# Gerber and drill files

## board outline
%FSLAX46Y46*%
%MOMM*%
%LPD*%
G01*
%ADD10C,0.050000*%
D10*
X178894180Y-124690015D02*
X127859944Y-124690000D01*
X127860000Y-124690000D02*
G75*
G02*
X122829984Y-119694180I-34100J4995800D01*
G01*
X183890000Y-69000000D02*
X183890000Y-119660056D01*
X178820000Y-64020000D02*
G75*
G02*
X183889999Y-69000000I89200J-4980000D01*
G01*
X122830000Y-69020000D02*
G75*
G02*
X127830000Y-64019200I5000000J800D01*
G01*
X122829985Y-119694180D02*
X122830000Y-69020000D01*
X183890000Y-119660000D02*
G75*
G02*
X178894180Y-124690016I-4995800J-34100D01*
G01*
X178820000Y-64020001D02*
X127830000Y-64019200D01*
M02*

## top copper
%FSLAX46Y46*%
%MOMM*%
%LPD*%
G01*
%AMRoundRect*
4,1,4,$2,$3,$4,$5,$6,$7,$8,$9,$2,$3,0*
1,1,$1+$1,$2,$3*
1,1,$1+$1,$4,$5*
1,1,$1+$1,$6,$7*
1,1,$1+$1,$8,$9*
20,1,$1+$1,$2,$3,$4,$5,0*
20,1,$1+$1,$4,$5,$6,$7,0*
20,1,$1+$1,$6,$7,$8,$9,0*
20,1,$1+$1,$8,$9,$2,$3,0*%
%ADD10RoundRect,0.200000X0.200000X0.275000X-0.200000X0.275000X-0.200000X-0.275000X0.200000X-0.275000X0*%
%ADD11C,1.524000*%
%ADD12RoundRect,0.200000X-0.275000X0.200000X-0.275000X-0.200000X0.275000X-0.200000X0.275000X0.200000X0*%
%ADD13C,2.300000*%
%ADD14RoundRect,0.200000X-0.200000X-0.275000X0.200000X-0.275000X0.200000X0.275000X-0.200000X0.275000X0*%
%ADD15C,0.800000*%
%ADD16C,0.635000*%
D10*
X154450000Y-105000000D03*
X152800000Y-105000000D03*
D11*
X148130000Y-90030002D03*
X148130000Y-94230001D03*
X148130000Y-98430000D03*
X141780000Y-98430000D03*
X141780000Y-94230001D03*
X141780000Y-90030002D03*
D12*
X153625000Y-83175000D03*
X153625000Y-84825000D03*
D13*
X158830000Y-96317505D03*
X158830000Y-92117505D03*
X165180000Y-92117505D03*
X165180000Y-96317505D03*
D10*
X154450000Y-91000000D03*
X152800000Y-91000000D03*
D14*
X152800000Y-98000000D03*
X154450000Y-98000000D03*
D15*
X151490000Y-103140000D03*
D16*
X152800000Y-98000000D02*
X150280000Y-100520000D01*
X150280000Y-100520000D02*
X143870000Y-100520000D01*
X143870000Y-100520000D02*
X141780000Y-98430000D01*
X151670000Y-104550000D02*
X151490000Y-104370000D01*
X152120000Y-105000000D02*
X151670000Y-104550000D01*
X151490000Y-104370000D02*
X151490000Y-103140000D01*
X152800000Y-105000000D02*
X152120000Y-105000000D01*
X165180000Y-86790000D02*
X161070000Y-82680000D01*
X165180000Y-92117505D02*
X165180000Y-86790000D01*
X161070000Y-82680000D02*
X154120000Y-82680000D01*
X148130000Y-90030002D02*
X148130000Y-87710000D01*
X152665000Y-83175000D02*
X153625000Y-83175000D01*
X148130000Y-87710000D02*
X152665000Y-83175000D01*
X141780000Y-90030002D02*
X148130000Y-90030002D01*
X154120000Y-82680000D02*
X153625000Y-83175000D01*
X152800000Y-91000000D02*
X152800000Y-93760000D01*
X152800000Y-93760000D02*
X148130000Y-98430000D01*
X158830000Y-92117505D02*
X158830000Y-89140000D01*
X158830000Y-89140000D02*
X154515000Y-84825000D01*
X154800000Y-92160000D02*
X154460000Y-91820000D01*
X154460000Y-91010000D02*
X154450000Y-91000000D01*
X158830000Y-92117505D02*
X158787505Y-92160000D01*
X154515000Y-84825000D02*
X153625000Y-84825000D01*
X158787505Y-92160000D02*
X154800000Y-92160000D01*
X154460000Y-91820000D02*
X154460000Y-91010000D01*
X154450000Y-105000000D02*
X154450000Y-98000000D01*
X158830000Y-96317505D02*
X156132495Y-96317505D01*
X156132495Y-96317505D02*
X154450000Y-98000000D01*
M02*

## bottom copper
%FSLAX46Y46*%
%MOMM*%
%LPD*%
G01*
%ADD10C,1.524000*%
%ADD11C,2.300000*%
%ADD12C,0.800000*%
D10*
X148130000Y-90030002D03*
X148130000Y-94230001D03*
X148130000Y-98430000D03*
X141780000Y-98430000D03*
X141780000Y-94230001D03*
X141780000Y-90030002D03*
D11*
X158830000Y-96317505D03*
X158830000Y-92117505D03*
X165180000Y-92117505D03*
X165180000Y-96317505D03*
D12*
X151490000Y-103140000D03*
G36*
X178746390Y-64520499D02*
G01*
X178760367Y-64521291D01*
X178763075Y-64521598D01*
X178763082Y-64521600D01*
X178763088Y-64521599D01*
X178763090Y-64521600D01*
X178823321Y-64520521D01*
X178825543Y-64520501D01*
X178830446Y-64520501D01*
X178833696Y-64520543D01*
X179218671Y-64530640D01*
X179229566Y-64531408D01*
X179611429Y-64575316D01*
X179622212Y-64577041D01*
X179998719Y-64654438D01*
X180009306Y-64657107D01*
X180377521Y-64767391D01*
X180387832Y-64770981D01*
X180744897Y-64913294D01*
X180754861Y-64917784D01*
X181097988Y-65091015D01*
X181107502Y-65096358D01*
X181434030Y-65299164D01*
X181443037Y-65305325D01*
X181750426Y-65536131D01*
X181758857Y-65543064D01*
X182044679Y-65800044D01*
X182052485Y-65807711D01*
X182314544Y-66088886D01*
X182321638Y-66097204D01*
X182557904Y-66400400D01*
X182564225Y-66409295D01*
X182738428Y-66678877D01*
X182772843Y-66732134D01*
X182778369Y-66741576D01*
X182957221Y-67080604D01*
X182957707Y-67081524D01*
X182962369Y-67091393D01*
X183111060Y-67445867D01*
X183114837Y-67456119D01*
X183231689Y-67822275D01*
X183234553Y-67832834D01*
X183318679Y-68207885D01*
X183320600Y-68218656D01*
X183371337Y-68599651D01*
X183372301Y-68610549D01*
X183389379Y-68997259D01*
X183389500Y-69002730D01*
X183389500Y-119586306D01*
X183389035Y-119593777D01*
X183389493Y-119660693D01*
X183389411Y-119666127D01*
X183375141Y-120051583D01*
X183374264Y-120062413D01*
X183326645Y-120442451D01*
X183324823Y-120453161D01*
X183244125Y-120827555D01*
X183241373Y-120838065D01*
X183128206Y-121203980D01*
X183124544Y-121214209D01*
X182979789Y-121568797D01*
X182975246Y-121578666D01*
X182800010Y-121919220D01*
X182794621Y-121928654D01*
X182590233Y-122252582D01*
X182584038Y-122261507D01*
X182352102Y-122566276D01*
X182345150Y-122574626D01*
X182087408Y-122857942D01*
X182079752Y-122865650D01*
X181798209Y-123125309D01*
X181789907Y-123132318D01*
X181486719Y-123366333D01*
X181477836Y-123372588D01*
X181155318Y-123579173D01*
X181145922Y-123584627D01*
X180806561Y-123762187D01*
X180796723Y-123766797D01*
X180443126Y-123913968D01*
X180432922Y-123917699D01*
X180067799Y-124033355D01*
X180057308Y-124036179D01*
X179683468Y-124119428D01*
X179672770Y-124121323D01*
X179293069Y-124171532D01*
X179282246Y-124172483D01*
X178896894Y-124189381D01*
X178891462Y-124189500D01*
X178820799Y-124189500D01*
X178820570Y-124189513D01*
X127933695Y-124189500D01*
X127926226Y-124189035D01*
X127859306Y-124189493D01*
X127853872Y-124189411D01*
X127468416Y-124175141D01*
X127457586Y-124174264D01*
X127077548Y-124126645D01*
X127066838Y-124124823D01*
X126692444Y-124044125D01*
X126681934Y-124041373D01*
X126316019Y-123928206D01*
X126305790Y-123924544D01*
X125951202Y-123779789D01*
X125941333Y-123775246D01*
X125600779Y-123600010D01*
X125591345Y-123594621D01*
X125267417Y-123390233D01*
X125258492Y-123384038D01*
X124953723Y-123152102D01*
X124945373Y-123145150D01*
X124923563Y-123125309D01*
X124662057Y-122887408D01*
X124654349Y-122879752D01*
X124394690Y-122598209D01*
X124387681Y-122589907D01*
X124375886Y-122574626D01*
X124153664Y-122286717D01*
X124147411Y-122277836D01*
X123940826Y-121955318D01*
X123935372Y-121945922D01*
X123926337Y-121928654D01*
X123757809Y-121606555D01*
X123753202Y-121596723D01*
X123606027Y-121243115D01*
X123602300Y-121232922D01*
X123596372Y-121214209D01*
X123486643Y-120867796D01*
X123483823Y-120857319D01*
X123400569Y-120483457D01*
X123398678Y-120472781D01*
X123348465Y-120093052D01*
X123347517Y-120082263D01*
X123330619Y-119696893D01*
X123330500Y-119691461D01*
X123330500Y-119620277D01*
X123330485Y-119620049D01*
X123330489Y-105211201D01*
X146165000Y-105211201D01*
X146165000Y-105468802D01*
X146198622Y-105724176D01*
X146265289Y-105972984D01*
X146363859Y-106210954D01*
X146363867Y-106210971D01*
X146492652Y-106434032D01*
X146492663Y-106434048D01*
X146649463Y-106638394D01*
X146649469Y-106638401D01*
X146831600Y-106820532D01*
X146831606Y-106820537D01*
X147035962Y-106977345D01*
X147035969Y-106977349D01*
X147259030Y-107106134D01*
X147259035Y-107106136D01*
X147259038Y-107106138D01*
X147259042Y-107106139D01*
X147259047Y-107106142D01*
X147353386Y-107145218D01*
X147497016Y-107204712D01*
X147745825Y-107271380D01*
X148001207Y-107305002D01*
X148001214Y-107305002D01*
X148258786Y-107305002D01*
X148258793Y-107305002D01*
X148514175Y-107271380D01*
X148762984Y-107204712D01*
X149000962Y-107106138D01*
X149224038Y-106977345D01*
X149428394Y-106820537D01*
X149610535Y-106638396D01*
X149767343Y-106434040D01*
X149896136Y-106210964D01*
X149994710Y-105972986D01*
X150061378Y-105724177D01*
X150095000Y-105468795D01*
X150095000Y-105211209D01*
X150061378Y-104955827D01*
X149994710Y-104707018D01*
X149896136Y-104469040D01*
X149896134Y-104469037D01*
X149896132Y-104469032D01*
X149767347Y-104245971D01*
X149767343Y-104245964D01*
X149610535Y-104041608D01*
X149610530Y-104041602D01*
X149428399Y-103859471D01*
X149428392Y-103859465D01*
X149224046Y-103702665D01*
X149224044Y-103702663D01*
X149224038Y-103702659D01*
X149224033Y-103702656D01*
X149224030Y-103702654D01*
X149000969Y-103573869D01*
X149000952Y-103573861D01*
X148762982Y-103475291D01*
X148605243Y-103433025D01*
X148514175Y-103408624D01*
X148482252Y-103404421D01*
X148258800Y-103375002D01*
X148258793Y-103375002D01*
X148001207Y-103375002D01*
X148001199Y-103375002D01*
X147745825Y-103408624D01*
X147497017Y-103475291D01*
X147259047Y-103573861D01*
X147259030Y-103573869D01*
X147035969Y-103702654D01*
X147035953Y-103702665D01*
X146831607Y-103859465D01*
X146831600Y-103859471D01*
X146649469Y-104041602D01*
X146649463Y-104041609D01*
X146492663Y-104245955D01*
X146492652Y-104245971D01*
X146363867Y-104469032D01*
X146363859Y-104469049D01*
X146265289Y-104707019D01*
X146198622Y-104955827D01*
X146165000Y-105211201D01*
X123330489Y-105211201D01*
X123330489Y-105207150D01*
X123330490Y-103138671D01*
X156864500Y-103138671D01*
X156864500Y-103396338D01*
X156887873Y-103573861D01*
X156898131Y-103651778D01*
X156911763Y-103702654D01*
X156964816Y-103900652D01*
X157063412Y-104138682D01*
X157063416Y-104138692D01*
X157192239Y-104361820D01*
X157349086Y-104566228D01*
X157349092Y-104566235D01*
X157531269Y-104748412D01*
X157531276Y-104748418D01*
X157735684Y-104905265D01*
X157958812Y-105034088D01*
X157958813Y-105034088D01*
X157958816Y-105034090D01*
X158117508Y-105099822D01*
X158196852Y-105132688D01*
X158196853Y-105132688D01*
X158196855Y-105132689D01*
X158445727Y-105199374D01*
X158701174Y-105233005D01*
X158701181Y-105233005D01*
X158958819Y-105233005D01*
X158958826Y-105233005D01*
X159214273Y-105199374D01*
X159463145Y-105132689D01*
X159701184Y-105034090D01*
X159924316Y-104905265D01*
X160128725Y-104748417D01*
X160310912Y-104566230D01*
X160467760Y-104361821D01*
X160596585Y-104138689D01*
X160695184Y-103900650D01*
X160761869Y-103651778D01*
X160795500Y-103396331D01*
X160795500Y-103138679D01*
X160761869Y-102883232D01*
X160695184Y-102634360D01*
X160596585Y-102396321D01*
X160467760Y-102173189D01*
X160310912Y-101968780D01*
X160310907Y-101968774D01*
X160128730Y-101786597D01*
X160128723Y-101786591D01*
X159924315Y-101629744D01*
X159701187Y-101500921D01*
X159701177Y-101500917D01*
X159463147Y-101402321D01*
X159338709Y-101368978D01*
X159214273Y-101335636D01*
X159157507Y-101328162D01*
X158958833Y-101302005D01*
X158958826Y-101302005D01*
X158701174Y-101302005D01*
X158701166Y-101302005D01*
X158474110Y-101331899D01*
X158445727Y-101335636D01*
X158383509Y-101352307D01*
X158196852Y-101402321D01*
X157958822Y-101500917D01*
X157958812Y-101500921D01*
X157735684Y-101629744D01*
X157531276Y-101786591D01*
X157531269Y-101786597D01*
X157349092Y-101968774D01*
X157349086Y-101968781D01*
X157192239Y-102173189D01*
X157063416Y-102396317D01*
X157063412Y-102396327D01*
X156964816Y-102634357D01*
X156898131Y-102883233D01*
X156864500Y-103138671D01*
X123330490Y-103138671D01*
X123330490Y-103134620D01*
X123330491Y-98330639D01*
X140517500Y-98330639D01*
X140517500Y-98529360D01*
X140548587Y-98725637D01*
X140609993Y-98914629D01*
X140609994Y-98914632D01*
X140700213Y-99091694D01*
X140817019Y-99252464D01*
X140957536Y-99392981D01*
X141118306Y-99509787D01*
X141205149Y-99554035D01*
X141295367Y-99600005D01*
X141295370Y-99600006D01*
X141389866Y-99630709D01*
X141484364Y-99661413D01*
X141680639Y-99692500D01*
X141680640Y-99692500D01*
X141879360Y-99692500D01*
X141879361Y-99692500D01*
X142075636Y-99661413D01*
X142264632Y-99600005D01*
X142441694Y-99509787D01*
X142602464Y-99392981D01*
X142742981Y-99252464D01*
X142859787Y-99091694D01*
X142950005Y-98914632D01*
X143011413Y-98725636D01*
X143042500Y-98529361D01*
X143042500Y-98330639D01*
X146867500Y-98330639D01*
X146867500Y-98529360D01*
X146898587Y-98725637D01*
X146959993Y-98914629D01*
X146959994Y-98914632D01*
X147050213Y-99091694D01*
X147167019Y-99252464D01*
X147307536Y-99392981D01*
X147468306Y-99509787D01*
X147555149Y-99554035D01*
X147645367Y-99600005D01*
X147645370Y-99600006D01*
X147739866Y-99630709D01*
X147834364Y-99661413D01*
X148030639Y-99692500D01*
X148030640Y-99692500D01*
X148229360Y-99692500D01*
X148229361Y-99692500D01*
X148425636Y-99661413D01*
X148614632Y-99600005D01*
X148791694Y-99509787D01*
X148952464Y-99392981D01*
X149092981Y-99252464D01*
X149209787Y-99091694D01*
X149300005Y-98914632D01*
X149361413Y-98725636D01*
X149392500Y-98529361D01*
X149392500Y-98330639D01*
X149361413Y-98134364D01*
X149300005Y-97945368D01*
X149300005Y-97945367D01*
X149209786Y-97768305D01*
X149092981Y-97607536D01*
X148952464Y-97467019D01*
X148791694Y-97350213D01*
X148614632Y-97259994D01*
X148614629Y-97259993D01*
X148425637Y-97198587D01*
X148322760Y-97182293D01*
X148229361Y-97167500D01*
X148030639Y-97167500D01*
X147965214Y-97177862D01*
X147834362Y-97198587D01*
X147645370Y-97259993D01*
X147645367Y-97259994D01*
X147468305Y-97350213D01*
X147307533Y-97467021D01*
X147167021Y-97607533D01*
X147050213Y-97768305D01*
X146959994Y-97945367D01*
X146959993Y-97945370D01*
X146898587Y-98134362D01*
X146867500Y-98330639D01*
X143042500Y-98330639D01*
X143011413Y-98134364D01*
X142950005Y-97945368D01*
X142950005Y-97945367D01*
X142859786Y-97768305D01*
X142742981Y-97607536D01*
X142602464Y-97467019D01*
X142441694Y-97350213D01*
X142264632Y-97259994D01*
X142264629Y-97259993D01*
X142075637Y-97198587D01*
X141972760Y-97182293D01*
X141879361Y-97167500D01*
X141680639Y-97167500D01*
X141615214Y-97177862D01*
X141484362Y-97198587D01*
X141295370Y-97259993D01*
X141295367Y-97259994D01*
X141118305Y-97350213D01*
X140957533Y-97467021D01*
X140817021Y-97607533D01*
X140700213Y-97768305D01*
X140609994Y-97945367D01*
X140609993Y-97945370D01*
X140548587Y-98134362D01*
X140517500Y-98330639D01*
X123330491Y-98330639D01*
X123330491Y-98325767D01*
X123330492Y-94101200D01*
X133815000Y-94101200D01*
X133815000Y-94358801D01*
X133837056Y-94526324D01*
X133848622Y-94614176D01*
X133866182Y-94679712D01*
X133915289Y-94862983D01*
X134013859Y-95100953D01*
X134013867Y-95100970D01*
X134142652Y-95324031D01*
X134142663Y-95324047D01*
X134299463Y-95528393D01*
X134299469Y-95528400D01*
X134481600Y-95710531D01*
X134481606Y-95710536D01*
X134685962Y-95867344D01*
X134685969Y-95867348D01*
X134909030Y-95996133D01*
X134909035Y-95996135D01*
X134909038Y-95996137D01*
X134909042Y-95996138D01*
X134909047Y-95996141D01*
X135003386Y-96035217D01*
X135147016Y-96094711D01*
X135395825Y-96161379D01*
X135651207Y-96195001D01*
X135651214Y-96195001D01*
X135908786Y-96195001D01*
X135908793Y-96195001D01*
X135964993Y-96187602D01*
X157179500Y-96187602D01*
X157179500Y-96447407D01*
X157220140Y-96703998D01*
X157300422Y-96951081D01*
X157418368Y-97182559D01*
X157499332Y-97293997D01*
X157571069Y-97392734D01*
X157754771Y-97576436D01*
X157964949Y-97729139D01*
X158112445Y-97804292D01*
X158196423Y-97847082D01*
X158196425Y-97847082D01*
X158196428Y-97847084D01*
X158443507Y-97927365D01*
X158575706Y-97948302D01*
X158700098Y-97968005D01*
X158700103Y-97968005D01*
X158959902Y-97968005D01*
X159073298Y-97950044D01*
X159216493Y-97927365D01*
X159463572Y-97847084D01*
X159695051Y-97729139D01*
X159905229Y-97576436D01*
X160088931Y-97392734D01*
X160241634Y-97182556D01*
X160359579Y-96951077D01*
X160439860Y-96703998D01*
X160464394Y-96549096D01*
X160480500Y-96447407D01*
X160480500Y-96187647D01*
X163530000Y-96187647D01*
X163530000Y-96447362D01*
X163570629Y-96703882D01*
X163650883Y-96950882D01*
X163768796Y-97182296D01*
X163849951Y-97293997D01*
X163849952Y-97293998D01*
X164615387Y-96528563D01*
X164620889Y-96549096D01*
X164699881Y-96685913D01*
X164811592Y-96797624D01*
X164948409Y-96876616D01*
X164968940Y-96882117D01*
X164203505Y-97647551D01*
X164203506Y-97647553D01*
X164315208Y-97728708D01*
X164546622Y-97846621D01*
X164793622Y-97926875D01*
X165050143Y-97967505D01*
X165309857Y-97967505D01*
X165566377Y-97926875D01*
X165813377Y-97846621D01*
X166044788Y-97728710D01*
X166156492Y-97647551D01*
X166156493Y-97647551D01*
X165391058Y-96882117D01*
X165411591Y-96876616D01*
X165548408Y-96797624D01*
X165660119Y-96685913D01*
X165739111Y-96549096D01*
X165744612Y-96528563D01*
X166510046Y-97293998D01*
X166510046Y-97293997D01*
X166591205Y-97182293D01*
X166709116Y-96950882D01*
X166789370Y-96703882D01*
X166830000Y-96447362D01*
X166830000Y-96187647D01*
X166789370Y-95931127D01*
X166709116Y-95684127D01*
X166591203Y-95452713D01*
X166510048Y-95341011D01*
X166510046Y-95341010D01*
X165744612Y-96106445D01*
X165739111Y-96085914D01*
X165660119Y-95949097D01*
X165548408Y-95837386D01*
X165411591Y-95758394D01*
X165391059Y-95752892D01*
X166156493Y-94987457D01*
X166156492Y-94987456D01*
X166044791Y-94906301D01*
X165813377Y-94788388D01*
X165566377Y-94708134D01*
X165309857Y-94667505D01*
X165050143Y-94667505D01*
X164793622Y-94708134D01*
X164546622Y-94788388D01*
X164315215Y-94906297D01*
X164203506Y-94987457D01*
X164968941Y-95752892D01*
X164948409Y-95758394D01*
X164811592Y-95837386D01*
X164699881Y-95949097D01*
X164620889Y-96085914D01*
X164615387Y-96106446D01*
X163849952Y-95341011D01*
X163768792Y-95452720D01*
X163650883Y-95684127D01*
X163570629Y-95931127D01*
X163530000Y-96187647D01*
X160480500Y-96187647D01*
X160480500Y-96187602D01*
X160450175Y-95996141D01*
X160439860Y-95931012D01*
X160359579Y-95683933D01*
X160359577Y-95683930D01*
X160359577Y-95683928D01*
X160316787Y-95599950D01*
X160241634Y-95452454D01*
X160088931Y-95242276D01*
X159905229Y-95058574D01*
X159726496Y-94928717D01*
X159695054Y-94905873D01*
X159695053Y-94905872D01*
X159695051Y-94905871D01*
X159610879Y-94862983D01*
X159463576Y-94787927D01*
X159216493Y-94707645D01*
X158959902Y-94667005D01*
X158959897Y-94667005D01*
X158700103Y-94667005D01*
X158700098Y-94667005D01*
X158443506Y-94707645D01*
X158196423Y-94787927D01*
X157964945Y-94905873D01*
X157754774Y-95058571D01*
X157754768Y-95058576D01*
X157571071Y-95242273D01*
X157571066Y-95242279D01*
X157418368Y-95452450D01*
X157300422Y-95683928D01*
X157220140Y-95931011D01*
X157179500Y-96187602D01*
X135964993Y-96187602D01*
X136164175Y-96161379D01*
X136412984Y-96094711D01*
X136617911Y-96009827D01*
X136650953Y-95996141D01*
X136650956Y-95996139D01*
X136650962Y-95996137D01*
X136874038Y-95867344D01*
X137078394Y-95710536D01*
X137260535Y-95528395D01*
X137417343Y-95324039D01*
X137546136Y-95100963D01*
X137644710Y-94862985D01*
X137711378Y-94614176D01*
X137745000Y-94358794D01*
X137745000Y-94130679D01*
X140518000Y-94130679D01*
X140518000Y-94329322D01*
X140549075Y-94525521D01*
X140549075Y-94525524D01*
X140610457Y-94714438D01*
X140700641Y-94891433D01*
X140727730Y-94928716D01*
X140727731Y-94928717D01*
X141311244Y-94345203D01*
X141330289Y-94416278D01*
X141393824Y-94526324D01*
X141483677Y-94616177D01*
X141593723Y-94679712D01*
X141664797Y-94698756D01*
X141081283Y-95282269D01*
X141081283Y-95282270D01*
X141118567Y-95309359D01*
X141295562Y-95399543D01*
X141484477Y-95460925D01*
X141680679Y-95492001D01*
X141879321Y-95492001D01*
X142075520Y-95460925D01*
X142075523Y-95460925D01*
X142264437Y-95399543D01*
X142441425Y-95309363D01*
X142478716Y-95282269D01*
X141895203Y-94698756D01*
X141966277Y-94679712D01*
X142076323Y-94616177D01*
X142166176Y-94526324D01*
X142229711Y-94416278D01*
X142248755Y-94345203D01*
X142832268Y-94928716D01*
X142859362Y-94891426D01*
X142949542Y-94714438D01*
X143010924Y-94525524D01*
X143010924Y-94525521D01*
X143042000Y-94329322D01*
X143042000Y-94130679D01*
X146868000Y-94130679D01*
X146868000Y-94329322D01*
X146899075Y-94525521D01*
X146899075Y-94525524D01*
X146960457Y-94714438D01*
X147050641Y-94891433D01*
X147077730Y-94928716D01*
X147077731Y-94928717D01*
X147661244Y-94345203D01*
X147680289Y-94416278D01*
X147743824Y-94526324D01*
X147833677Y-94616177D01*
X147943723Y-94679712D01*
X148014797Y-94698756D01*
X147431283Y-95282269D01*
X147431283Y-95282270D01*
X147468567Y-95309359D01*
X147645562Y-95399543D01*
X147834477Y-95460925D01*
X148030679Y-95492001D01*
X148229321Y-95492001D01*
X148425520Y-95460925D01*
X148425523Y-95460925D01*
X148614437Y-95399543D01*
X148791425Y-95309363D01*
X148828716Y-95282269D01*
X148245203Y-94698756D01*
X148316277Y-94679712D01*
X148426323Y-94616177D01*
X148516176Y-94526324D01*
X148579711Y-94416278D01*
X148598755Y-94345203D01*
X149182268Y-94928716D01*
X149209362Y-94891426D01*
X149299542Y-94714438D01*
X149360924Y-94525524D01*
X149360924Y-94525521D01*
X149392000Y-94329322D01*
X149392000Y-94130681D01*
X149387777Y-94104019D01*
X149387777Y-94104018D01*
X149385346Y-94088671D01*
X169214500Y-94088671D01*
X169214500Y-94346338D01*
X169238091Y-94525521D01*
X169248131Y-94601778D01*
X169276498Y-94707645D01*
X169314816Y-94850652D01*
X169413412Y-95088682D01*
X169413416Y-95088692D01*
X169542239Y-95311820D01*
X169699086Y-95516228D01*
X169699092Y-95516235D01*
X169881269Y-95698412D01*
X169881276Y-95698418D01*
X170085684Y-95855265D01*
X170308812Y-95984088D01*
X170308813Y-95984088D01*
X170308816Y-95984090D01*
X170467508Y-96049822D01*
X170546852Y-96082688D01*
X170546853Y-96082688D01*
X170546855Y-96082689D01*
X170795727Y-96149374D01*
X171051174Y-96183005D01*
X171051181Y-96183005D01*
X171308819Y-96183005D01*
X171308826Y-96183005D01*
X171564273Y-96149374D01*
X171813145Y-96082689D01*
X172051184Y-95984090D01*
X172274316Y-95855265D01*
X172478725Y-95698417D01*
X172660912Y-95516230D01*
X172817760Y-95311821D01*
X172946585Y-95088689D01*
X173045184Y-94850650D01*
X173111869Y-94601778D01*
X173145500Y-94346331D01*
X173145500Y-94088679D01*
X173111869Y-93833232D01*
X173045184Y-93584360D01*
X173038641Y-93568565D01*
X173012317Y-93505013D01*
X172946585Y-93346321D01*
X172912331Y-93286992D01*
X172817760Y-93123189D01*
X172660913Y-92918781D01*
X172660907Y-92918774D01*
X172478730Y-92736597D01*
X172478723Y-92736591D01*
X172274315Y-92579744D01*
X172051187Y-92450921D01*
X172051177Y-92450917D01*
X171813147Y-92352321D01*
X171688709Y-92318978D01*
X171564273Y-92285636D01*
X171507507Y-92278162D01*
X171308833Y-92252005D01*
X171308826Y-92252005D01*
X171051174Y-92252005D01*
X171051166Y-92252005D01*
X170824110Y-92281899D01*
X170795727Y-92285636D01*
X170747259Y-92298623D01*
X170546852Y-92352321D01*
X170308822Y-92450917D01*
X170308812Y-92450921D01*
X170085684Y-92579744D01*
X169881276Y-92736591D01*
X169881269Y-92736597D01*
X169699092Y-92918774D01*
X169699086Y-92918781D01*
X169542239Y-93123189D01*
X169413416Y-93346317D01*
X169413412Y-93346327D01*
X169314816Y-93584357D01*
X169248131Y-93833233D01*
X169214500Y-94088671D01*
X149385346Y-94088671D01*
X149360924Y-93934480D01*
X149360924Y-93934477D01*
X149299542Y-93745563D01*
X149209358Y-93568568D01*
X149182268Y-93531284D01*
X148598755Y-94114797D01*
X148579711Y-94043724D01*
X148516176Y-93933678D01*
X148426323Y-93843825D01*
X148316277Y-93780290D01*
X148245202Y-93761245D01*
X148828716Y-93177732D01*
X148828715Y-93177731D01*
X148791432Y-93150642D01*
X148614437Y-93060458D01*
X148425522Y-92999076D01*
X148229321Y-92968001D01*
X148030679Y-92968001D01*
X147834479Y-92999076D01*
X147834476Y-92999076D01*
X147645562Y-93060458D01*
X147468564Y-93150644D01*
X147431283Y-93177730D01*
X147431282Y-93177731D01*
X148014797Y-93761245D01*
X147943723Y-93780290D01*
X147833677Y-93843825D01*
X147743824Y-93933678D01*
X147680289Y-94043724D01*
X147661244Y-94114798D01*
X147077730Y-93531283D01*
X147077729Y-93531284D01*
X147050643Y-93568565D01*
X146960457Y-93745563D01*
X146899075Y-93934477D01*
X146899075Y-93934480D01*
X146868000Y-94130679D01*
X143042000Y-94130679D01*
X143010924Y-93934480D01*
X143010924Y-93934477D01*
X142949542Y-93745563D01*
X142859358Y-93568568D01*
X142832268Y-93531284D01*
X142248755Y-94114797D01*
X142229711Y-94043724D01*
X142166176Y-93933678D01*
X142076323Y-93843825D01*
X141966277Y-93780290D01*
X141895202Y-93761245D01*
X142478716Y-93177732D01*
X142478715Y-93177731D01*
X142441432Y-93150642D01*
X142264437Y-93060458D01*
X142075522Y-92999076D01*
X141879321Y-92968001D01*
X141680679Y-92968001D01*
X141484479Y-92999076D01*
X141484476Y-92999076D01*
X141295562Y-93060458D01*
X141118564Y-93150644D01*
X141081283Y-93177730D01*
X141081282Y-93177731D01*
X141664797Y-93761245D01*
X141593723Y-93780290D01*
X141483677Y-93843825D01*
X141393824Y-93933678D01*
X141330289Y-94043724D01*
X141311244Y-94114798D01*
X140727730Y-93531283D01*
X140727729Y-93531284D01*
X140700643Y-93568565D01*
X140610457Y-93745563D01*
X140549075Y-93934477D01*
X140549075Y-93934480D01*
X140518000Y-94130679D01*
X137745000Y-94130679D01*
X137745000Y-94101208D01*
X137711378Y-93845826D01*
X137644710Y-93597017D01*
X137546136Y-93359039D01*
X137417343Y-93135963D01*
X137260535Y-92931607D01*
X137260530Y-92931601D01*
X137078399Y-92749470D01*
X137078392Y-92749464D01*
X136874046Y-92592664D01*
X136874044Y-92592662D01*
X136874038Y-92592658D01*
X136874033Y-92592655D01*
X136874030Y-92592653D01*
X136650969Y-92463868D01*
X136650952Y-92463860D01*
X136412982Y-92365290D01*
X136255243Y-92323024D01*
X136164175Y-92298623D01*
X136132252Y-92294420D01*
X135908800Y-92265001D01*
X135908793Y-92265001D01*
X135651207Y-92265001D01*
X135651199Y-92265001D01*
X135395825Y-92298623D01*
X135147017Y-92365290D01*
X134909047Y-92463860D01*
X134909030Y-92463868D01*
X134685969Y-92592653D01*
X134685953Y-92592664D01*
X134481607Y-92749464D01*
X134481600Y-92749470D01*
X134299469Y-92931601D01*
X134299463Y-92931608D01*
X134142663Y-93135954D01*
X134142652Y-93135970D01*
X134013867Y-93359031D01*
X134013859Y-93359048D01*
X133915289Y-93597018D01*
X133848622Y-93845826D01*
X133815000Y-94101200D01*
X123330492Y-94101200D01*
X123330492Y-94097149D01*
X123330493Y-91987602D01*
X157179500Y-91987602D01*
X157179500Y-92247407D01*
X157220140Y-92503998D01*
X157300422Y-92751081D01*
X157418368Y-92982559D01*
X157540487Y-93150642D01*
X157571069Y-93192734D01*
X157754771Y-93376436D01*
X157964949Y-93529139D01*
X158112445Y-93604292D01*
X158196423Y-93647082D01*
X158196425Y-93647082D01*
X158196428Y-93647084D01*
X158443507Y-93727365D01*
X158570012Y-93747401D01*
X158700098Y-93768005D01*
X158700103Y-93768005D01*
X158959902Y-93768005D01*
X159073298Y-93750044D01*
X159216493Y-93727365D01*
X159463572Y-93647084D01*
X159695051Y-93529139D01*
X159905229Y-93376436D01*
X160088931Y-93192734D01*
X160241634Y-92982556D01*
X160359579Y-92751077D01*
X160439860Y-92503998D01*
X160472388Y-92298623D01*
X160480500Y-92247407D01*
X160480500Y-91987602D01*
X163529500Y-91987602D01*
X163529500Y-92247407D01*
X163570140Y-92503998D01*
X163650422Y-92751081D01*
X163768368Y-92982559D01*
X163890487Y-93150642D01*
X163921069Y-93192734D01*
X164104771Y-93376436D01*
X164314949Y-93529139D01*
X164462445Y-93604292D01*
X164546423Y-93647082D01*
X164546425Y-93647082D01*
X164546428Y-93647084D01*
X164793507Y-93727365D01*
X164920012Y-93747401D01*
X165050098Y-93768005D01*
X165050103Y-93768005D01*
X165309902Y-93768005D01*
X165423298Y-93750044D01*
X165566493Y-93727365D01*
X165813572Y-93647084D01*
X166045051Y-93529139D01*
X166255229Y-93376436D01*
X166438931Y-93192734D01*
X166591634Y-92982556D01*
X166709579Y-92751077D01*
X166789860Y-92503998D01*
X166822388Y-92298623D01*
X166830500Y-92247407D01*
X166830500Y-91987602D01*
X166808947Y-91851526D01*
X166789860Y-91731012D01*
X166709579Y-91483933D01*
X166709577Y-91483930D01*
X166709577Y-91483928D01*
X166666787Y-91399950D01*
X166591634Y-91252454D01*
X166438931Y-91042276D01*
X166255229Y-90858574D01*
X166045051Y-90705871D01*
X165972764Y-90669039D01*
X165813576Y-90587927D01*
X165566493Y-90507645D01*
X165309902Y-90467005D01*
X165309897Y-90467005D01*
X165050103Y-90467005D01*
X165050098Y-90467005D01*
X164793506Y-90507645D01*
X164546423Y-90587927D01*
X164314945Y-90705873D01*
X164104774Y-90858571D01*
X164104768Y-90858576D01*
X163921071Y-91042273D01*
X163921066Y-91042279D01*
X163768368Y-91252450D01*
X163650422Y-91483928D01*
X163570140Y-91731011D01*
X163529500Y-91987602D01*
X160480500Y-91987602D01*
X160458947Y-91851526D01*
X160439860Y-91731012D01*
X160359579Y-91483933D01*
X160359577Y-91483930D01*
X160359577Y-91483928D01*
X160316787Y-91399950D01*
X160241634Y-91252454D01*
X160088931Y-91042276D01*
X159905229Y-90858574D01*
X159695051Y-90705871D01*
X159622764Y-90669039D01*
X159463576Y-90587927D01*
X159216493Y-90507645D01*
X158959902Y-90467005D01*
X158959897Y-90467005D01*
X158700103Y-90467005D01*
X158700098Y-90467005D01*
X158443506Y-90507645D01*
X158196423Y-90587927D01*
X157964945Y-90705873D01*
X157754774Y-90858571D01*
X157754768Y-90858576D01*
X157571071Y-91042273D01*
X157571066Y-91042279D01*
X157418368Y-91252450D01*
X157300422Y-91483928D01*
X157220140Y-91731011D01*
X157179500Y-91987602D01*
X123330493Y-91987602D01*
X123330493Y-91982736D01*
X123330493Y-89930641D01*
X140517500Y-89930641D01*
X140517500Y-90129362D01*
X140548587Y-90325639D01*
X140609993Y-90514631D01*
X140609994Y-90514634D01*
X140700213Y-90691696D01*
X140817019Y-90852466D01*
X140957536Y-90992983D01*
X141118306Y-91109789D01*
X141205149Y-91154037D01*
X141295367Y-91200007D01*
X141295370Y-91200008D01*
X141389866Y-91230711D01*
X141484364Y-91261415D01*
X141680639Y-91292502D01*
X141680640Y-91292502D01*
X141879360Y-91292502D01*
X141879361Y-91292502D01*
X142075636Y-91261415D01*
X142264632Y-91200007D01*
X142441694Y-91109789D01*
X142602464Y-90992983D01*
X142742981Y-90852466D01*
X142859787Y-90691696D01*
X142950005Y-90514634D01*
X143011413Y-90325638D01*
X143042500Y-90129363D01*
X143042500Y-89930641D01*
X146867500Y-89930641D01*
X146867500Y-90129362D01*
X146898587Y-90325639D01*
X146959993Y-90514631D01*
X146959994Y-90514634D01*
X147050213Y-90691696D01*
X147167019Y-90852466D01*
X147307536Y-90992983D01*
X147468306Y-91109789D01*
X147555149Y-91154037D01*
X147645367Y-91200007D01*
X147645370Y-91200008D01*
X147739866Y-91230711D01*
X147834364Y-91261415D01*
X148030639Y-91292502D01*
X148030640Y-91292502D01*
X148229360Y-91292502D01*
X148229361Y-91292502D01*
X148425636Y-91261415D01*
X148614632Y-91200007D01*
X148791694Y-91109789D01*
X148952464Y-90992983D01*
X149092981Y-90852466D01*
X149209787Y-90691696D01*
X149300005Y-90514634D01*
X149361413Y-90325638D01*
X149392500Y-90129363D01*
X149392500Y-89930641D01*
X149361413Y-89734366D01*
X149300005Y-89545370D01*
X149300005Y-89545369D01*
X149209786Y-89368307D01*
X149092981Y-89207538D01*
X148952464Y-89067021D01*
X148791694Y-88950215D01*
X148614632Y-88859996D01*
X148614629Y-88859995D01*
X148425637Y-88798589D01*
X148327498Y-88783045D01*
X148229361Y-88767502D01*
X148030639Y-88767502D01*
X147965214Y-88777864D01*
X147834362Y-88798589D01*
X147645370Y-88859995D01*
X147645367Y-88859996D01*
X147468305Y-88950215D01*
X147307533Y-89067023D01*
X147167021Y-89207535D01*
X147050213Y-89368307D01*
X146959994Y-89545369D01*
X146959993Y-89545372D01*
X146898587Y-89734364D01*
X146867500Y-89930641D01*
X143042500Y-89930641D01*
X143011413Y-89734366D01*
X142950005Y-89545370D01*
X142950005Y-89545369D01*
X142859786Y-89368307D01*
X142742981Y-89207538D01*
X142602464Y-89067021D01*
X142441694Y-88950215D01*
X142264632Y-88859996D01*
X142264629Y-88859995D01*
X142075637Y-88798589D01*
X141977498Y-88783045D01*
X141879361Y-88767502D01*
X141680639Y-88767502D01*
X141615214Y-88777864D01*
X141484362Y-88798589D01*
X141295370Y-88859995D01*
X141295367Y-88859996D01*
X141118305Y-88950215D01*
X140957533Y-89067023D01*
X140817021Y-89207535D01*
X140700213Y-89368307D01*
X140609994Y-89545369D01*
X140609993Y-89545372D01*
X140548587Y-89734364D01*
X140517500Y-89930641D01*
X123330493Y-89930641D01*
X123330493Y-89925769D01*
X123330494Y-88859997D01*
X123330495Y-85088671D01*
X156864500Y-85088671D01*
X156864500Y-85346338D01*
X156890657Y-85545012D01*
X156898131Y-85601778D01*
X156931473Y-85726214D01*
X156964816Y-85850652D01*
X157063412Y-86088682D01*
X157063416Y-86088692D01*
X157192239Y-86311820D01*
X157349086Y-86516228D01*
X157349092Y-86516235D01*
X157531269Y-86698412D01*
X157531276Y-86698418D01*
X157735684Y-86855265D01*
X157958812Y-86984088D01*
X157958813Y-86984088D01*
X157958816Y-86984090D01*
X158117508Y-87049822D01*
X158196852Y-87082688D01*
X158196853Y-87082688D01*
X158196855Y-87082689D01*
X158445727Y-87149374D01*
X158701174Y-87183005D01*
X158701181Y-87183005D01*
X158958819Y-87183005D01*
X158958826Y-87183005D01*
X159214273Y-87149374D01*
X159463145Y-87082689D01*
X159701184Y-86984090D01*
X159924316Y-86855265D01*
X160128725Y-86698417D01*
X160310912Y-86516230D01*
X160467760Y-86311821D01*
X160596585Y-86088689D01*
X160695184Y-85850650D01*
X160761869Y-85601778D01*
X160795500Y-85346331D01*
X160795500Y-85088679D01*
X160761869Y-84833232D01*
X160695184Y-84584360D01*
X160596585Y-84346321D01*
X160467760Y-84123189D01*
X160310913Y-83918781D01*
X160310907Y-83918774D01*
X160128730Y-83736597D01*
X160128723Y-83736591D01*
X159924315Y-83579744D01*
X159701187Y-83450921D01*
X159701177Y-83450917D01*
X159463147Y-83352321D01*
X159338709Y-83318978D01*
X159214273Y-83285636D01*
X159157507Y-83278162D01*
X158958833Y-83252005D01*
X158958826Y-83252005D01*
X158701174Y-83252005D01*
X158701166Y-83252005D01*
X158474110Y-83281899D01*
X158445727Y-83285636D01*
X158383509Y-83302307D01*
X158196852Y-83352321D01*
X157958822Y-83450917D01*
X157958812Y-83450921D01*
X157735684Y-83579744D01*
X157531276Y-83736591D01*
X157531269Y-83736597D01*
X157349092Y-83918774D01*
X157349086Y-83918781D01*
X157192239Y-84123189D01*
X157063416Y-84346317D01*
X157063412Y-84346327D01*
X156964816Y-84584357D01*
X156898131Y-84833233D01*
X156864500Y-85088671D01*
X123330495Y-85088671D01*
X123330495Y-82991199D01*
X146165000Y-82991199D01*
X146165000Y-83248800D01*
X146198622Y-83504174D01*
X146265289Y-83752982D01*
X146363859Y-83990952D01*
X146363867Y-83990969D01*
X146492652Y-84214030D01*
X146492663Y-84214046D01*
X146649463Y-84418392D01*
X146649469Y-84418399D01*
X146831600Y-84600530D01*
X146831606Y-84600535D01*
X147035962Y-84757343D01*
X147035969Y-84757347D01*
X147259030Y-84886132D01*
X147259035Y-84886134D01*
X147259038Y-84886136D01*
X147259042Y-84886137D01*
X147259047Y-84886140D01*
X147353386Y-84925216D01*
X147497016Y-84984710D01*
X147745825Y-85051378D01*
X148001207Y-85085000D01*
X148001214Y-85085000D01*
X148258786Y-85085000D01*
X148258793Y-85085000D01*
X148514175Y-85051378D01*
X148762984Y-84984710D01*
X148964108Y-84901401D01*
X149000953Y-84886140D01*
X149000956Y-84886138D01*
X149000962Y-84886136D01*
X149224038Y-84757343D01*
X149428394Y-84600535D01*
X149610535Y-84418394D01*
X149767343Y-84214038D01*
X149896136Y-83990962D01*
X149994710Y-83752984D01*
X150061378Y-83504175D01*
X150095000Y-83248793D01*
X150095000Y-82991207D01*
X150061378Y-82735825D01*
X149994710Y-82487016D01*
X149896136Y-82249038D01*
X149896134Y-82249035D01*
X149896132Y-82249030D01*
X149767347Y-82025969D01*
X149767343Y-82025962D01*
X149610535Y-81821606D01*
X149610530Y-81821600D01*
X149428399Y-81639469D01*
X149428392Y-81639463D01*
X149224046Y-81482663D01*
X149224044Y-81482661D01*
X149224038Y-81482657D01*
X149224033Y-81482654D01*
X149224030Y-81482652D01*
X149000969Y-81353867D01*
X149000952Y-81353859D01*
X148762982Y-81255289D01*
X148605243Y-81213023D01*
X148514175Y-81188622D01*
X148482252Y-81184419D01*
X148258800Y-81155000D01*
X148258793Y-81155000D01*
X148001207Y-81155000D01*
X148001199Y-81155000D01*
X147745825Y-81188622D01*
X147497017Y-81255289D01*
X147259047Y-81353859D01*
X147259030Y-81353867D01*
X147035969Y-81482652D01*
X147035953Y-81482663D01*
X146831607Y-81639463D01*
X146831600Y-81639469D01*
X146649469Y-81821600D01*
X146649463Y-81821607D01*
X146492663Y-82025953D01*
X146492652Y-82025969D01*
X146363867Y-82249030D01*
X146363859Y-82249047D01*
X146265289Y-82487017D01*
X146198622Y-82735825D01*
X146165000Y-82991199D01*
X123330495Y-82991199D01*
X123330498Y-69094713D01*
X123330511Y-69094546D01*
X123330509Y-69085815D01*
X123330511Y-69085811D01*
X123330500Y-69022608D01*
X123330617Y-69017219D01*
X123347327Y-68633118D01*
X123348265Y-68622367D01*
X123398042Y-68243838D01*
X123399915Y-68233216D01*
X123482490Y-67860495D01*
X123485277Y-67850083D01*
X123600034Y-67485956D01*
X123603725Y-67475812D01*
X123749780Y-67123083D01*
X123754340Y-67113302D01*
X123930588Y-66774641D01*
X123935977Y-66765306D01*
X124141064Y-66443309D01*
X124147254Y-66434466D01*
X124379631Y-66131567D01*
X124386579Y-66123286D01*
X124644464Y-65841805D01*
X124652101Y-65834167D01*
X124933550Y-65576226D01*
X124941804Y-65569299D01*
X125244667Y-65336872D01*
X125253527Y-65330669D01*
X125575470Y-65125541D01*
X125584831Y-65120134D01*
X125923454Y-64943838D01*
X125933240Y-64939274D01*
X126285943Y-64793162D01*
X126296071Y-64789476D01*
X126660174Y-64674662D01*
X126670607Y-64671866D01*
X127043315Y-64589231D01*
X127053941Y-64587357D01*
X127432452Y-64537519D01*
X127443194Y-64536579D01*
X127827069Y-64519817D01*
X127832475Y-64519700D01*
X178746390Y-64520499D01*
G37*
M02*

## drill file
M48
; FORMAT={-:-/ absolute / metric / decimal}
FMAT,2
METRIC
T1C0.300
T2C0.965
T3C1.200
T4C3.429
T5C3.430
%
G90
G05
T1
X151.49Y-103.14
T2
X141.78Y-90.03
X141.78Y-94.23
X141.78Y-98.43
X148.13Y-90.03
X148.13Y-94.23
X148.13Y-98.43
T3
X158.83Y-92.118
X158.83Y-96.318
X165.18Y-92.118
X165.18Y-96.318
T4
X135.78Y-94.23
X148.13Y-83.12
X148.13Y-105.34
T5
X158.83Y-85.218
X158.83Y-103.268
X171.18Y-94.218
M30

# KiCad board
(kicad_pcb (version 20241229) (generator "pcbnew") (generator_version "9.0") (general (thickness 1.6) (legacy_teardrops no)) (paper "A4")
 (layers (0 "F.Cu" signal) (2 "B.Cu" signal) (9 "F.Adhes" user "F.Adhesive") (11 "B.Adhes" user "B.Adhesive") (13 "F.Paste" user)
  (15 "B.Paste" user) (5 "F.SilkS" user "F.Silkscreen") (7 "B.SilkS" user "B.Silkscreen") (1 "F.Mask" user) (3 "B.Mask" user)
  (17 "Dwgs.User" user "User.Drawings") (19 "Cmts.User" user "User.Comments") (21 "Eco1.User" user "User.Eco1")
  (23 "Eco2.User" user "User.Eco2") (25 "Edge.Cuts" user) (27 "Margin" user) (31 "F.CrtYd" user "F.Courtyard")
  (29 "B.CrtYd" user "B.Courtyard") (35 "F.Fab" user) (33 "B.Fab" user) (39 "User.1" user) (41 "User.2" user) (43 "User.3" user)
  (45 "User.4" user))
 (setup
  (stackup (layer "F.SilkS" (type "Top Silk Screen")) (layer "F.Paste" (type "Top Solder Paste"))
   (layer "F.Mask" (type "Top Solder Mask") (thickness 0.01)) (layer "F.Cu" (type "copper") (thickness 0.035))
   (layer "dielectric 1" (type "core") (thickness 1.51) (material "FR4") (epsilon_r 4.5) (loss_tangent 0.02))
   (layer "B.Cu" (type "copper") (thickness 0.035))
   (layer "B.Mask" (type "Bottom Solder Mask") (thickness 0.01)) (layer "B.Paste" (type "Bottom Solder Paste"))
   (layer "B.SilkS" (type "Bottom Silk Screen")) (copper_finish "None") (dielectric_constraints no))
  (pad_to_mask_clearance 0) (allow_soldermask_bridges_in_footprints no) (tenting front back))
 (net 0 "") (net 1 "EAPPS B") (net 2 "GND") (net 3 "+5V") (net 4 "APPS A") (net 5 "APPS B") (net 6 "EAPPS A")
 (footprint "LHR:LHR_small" (layer "F.Cu") (at 172.32 118.24)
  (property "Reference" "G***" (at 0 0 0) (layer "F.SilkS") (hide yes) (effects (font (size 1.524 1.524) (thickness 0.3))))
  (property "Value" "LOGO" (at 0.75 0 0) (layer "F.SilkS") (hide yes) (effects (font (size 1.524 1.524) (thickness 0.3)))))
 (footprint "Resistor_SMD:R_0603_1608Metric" (layer "F.Cu") (at 153.625 105 180)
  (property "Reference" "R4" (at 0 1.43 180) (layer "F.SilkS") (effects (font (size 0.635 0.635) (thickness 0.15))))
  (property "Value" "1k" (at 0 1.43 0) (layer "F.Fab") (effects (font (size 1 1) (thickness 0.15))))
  (pad "1" smd roundrect (at -0.825 0 180) (size 0.8 0.95) (layers "F.Cu" "F.Mask" "F.Paste") (roundrect_rratio 0.25) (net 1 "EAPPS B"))
  (pad "2" smd roundrect (at 0.825 0 180) (size 0.8 0.95) (layers "F.Cu" "F.Mask" "F.Paste") (roundrect_rratio 0.25) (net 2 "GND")))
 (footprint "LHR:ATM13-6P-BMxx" (layer "F.Cu") (at 148.13 90.030002 -90)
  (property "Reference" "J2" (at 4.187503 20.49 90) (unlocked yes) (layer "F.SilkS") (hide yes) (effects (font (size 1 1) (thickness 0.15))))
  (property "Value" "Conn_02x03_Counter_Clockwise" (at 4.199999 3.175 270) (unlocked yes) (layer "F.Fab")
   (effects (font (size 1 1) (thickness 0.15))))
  (pad "" np_thru_hole circle (at -6.910002 0 270) (size 3.937 3.937) (drill 3.429) (layers))
  (pad "" np_thru_hole circle (at 4.199999 12.35 270) (size 3.937 3.937) (drill 3.429) (layers))
  (pad "" np_thru_hole circle (at 15.31 0 270) (size 3.937 3.937) (drill 3.429) (layers))
  (pad "1" thru_hole circle (at 0 0 270) (size 1.524 1.524) (drill 0.9652) (layers "*.Cu" "*.Mask") (remove_unused_layers no) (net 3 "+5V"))
  (pad "2" thru_hole circle (at 4.199999 0 270) (size 1.524 1.524) (drill 0.9652) (layers "*.Cu" "*.Mask") (remove_unused_layers no)
   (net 2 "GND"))
  (pad "3" thru_hole circle (at 8.399998 0 270) (size 1.524 1.524) (drill 0.9652) (layers "*.Cu" "*.Mask") (remove_unused_layers no)
   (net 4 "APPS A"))
  (pad "4" thru_hole circle (at 8.399998 6.35 270) (size 1.524 1.524) (drill 0.9652) (layers "*.Cu" "*.Mask") (remove_unused_layers no)
   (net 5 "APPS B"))
  (pad "5" thru_hole circle (at 4.199999 6.35 270) (size 1.524 1.524) (drill 0.9652) (layers "*.Cu" "*.Mask") (remove_unused_layers no)
   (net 2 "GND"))
  (pad "6" thru_hole circle (at 0 6.35 270) (size 1.524 1.524) (drill 0.9652) (layers "*.Cu" "*.Mask") (remove_unused_layers no)
   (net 3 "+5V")))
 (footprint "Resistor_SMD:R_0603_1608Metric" (layer "F.Cu") (at 153.625 84 -90)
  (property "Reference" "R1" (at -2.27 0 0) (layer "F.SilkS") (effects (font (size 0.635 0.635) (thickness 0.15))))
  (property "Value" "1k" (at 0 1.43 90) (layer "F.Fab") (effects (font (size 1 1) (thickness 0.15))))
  (pad "1" smd roundrect (at -0.825 0 270) (size 0.8 0.95) (layers "F.Cu" "F.Mask" "F.Paste") (roundrect_rratio 0.25) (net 3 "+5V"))
  (pad "2" smd roundrect (at 0.825 0 270) (size 0.8 0.95) (layers "F.Cu" "F.Mask" "F.Paste") (roundrect_rratio 0.25) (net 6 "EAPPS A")))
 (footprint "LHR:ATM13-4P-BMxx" (layer "F.Cu") (at 164.08 94.217505 -90)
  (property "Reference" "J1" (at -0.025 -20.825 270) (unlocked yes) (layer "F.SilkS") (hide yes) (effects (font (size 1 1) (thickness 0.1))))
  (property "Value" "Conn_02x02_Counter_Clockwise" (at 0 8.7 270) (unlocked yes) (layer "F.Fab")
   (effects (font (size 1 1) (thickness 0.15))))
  (pad "" np_thru_hole circle (at -9 5.25 270) (size 3.43 3.43) (drill 3.43) (layers "*.Cu" "*.Mask"))
  (pad "" np_thru_hole circle (at 0 -7.1 270) (size 3.43 3.43) (drill 3.43) (layers "*.Cu" "*.Mask"))
  (pad "" np_thru_hole circle (at 9.05 5.25 270) (size 3.43 3.43) (drill 3.43) (layers "*.Cu" "*.Mask"))
  (pad "1" thru_hole circle (at 2.1 5.25 270) (size 2.3 2.3) (drill 1.2) (layers "*.Cu" "*.Mask") (remove_unused_layers no)
   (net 1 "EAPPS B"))
  (pad "2" thru_hole circle (at -2.1 5.25 270) (size 2.3 2.3) (drill 1.2) (layers "*.Cu" "*.Mask") (remove_unused_layers no)
   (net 6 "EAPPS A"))
  (pad "3" thru_hole circle (at -2.1 -1.1 270) (size 2.3 2.3) (drill 1.2) (layers "*.Cu" "*.Mask") (remove_unused_layers no) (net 3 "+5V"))
  (pad "4" thru_hole circle (at 2.1 -1.1 270) (size 2.3 2.3) (drill 1.2) (layers "*.Cu" "*.Mask") (remove_unused_layers no) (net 2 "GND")))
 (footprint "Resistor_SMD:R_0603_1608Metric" (layer "F.Cu") (at 153.625 91 180)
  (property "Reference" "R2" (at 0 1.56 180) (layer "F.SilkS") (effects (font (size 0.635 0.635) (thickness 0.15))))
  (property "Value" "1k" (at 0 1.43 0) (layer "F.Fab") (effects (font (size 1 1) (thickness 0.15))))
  (pad "1" smd roundrect (at -0.825 0 180) (size 0.8 0.95) (layers "F.Cu" "F.Mask" "F.Paste") (roundrect_rratio 0.25) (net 6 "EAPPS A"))
  (pad "2" smd roundrect (at 0.825 0 180) (size 0.8 0.95) (layers "F.Cu" "F.Mask" "F.Paste") (roundrect_rratio 0.25) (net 4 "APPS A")))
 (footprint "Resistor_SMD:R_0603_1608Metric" (layer "F.Cu") (at 153.625 98)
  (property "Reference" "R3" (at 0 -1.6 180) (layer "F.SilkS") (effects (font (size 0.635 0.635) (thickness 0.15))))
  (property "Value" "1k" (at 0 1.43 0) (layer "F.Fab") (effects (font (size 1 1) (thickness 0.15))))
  (pad "1" smd roundrect (at -0.825 0) (size 0.8 0.95) (layers "F.Cu" "F.Mask" "F.Paste") (roundrect_rratio 0.25) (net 5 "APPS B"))
  (pad "2" smd roundrect (at 0.825 0) (size 0.8 0.95) (layers "F.Cu" "F.Mask" "F.Paste") (roundrect_rratio 0.25) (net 1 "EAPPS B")))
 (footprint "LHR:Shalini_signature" (layer "B.Cu") (at 170.92 71.88 180)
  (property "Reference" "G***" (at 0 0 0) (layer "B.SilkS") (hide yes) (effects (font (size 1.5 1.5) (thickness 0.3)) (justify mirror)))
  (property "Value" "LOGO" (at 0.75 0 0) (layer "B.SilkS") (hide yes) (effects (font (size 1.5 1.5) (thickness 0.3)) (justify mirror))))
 (gr_line (start 178.89418 124.690015) (end 127.859944 124.69) (stroke (width 0.05) (type default)) (layer "Edge.Cuts"))
 (gr_arc (start 127.86 124.69) (mid 124.30534 123.238863) (end 122.83 119.69418) (stroke (width 0.05) (type default)) (layer "Edge.Cuts"))
 (gr_line (start 183.89 69) (end 183.89 119.660056) (stroke (width 0.05) (type default)) (layer "Edge.Cuts"))
 (gr_arc (start 178.82 64.02) (mid 182.399478 65.446646) (end 183.89 69) (stroke (width 0.05) (type default)) (layer "Edge.Cuts"))
 (gr_arc (start 122.83 69.02) (mid 124.29418 65.483942) (end 127.83 64.01919) (stroke (width 0.05) (type default)) (layer "Edge.Cuts"))
 (gr_line (start 122.829985 119.69418) (end 122.83 69.02) (stroke (width 0.05) (type default)) (layer "Edge.Cuts"))
 (gr_arc (start 183.89 119.66) (mid 182.438863 123.21466) (end 178.89418 124.69) (stroke (width 0.05) (type default)) (layer "Edge.Cuts"))
 (gr_line (start 178.82 64.020001) (end 127.83 64.0192) (stroke (width 0.05) (type default)) (layer "Edge.Cuts"))
 (segment (start 152.8 98) (end 150.28 100.52) (width 0.635) (layer "F.Cu") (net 5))
 (segment (start 150.28 100.52) (end 143.87 100.52) (width 0.635) (layer "F.Cu") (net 5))
 (segment (start 143.87 100.52) (end 141.78 98.43) (width 0.635) (layer "F.Cu") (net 5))
 (segment (start 151.67 104.55) (end 151.49 104.37) (width 0.635) (layer "F.Cu") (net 2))
 (segment (start 152.12 105) (end 151.67 104.55) (width 0.635) (layer "F.Cu") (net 2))
 (segment (start 151.49 104.37) (end 151.49 103.14) (width 0.635) (layer "F.Cu") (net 2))
 (segment (start 152.8 105) (end 152.12 105) (width 0.635) (layer "F.Cu") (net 2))
 (via (at 151.49 103.14) (size 0.8) (drill 0.3) (layers "F.Cu" "B.Cu") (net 2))
 (segment (start 165.18 86.79) (end 161.07 82.68) (width 0.635) (layer "F.Cu") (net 3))
 (segment (start 165.18 92.117505) (end 165.18 86.79) (width 0.635) (layer "F.Cu") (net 3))
 (segment (start 161.07 82.68) (end 154.12 82.68) (width 0.635) (layer "F.Cu") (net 3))
 (segment (start 148.13 90.030002) (end 148.13 87.71) (width 0.635) (layer "F.Cu") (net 3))
 (segment (start 152.665 83.175) (end 153.625 83.175) (width 0.635) (layer "F.Cu") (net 3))
 (segment (start 148.13 87.71) (end 152.665 83.175) (width 0.635) (layer "F.Cu") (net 3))
 (segment (start 141.78 90.030002) (end 148.13 90.030002) (width 0.635) (layer "F.Cu") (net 3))
 (segment (start 154.12 82.68) (end 153.625 83.175) (width 0.635) (layer "F.Cu") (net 3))
 (segment (start 152.8 91) (end 152.8 93.76) (width 0.635) (layer "F.Cu") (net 4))
 (segment (start 152.8 93.76) (end 148.13 98.43) (width 0.635) (layer "F.Cu") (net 4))
 (segment (start 158.83 92.117505) (end 158.83 89.14) (width 0.635) (layer "F.Cu") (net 6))
 (segment (start 158.83 89.14) (end 154.515 84.825) (width 0.635) (layer "F.Cu") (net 6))
 (segment (start 154.8 92.16) (end 154.46 91.82) (width 0.635) (layer "F.Cu") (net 6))
 (segment (start 154.46 91.01) (end 154.45 91) (width 0.635) (layer "F.Cu") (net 6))
 (segment (start 158.83 92.117505) (end 158.787505 92.16) (width 0.635) (layer "F.Cu") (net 6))
 (segment (start 154.515 84.825) (end 153.625 84.825) (width 0.635) (layer "F.Cu") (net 6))
 (segment (start 158.787505 92.16) (end 154.8 92.16) (width 0.635) (layer "F.Cu") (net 6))
 (segment (start 154.46 91.82) (end 154.46 91.01) (width 0.635) (layer "F.Cu") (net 6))
 (segment (start 154.45 105) (end 154.45 98) (width 0.635) (layer "F.Cu") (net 1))
 (segment (start 158.83 96.317505) (end 156.132495 96.317505) (width 0.635) (layer "F.Cu") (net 1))
 (segment (start 156.132495 96.317505) (end 154.45 98) (width 0.635) (layer "F.Cu") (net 1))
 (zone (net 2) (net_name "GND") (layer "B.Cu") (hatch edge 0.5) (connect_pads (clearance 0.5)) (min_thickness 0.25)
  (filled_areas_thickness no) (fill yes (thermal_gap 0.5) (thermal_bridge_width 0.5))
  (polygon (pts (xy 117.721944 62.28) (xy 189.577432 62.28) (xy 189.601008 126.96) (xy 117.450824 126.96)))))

